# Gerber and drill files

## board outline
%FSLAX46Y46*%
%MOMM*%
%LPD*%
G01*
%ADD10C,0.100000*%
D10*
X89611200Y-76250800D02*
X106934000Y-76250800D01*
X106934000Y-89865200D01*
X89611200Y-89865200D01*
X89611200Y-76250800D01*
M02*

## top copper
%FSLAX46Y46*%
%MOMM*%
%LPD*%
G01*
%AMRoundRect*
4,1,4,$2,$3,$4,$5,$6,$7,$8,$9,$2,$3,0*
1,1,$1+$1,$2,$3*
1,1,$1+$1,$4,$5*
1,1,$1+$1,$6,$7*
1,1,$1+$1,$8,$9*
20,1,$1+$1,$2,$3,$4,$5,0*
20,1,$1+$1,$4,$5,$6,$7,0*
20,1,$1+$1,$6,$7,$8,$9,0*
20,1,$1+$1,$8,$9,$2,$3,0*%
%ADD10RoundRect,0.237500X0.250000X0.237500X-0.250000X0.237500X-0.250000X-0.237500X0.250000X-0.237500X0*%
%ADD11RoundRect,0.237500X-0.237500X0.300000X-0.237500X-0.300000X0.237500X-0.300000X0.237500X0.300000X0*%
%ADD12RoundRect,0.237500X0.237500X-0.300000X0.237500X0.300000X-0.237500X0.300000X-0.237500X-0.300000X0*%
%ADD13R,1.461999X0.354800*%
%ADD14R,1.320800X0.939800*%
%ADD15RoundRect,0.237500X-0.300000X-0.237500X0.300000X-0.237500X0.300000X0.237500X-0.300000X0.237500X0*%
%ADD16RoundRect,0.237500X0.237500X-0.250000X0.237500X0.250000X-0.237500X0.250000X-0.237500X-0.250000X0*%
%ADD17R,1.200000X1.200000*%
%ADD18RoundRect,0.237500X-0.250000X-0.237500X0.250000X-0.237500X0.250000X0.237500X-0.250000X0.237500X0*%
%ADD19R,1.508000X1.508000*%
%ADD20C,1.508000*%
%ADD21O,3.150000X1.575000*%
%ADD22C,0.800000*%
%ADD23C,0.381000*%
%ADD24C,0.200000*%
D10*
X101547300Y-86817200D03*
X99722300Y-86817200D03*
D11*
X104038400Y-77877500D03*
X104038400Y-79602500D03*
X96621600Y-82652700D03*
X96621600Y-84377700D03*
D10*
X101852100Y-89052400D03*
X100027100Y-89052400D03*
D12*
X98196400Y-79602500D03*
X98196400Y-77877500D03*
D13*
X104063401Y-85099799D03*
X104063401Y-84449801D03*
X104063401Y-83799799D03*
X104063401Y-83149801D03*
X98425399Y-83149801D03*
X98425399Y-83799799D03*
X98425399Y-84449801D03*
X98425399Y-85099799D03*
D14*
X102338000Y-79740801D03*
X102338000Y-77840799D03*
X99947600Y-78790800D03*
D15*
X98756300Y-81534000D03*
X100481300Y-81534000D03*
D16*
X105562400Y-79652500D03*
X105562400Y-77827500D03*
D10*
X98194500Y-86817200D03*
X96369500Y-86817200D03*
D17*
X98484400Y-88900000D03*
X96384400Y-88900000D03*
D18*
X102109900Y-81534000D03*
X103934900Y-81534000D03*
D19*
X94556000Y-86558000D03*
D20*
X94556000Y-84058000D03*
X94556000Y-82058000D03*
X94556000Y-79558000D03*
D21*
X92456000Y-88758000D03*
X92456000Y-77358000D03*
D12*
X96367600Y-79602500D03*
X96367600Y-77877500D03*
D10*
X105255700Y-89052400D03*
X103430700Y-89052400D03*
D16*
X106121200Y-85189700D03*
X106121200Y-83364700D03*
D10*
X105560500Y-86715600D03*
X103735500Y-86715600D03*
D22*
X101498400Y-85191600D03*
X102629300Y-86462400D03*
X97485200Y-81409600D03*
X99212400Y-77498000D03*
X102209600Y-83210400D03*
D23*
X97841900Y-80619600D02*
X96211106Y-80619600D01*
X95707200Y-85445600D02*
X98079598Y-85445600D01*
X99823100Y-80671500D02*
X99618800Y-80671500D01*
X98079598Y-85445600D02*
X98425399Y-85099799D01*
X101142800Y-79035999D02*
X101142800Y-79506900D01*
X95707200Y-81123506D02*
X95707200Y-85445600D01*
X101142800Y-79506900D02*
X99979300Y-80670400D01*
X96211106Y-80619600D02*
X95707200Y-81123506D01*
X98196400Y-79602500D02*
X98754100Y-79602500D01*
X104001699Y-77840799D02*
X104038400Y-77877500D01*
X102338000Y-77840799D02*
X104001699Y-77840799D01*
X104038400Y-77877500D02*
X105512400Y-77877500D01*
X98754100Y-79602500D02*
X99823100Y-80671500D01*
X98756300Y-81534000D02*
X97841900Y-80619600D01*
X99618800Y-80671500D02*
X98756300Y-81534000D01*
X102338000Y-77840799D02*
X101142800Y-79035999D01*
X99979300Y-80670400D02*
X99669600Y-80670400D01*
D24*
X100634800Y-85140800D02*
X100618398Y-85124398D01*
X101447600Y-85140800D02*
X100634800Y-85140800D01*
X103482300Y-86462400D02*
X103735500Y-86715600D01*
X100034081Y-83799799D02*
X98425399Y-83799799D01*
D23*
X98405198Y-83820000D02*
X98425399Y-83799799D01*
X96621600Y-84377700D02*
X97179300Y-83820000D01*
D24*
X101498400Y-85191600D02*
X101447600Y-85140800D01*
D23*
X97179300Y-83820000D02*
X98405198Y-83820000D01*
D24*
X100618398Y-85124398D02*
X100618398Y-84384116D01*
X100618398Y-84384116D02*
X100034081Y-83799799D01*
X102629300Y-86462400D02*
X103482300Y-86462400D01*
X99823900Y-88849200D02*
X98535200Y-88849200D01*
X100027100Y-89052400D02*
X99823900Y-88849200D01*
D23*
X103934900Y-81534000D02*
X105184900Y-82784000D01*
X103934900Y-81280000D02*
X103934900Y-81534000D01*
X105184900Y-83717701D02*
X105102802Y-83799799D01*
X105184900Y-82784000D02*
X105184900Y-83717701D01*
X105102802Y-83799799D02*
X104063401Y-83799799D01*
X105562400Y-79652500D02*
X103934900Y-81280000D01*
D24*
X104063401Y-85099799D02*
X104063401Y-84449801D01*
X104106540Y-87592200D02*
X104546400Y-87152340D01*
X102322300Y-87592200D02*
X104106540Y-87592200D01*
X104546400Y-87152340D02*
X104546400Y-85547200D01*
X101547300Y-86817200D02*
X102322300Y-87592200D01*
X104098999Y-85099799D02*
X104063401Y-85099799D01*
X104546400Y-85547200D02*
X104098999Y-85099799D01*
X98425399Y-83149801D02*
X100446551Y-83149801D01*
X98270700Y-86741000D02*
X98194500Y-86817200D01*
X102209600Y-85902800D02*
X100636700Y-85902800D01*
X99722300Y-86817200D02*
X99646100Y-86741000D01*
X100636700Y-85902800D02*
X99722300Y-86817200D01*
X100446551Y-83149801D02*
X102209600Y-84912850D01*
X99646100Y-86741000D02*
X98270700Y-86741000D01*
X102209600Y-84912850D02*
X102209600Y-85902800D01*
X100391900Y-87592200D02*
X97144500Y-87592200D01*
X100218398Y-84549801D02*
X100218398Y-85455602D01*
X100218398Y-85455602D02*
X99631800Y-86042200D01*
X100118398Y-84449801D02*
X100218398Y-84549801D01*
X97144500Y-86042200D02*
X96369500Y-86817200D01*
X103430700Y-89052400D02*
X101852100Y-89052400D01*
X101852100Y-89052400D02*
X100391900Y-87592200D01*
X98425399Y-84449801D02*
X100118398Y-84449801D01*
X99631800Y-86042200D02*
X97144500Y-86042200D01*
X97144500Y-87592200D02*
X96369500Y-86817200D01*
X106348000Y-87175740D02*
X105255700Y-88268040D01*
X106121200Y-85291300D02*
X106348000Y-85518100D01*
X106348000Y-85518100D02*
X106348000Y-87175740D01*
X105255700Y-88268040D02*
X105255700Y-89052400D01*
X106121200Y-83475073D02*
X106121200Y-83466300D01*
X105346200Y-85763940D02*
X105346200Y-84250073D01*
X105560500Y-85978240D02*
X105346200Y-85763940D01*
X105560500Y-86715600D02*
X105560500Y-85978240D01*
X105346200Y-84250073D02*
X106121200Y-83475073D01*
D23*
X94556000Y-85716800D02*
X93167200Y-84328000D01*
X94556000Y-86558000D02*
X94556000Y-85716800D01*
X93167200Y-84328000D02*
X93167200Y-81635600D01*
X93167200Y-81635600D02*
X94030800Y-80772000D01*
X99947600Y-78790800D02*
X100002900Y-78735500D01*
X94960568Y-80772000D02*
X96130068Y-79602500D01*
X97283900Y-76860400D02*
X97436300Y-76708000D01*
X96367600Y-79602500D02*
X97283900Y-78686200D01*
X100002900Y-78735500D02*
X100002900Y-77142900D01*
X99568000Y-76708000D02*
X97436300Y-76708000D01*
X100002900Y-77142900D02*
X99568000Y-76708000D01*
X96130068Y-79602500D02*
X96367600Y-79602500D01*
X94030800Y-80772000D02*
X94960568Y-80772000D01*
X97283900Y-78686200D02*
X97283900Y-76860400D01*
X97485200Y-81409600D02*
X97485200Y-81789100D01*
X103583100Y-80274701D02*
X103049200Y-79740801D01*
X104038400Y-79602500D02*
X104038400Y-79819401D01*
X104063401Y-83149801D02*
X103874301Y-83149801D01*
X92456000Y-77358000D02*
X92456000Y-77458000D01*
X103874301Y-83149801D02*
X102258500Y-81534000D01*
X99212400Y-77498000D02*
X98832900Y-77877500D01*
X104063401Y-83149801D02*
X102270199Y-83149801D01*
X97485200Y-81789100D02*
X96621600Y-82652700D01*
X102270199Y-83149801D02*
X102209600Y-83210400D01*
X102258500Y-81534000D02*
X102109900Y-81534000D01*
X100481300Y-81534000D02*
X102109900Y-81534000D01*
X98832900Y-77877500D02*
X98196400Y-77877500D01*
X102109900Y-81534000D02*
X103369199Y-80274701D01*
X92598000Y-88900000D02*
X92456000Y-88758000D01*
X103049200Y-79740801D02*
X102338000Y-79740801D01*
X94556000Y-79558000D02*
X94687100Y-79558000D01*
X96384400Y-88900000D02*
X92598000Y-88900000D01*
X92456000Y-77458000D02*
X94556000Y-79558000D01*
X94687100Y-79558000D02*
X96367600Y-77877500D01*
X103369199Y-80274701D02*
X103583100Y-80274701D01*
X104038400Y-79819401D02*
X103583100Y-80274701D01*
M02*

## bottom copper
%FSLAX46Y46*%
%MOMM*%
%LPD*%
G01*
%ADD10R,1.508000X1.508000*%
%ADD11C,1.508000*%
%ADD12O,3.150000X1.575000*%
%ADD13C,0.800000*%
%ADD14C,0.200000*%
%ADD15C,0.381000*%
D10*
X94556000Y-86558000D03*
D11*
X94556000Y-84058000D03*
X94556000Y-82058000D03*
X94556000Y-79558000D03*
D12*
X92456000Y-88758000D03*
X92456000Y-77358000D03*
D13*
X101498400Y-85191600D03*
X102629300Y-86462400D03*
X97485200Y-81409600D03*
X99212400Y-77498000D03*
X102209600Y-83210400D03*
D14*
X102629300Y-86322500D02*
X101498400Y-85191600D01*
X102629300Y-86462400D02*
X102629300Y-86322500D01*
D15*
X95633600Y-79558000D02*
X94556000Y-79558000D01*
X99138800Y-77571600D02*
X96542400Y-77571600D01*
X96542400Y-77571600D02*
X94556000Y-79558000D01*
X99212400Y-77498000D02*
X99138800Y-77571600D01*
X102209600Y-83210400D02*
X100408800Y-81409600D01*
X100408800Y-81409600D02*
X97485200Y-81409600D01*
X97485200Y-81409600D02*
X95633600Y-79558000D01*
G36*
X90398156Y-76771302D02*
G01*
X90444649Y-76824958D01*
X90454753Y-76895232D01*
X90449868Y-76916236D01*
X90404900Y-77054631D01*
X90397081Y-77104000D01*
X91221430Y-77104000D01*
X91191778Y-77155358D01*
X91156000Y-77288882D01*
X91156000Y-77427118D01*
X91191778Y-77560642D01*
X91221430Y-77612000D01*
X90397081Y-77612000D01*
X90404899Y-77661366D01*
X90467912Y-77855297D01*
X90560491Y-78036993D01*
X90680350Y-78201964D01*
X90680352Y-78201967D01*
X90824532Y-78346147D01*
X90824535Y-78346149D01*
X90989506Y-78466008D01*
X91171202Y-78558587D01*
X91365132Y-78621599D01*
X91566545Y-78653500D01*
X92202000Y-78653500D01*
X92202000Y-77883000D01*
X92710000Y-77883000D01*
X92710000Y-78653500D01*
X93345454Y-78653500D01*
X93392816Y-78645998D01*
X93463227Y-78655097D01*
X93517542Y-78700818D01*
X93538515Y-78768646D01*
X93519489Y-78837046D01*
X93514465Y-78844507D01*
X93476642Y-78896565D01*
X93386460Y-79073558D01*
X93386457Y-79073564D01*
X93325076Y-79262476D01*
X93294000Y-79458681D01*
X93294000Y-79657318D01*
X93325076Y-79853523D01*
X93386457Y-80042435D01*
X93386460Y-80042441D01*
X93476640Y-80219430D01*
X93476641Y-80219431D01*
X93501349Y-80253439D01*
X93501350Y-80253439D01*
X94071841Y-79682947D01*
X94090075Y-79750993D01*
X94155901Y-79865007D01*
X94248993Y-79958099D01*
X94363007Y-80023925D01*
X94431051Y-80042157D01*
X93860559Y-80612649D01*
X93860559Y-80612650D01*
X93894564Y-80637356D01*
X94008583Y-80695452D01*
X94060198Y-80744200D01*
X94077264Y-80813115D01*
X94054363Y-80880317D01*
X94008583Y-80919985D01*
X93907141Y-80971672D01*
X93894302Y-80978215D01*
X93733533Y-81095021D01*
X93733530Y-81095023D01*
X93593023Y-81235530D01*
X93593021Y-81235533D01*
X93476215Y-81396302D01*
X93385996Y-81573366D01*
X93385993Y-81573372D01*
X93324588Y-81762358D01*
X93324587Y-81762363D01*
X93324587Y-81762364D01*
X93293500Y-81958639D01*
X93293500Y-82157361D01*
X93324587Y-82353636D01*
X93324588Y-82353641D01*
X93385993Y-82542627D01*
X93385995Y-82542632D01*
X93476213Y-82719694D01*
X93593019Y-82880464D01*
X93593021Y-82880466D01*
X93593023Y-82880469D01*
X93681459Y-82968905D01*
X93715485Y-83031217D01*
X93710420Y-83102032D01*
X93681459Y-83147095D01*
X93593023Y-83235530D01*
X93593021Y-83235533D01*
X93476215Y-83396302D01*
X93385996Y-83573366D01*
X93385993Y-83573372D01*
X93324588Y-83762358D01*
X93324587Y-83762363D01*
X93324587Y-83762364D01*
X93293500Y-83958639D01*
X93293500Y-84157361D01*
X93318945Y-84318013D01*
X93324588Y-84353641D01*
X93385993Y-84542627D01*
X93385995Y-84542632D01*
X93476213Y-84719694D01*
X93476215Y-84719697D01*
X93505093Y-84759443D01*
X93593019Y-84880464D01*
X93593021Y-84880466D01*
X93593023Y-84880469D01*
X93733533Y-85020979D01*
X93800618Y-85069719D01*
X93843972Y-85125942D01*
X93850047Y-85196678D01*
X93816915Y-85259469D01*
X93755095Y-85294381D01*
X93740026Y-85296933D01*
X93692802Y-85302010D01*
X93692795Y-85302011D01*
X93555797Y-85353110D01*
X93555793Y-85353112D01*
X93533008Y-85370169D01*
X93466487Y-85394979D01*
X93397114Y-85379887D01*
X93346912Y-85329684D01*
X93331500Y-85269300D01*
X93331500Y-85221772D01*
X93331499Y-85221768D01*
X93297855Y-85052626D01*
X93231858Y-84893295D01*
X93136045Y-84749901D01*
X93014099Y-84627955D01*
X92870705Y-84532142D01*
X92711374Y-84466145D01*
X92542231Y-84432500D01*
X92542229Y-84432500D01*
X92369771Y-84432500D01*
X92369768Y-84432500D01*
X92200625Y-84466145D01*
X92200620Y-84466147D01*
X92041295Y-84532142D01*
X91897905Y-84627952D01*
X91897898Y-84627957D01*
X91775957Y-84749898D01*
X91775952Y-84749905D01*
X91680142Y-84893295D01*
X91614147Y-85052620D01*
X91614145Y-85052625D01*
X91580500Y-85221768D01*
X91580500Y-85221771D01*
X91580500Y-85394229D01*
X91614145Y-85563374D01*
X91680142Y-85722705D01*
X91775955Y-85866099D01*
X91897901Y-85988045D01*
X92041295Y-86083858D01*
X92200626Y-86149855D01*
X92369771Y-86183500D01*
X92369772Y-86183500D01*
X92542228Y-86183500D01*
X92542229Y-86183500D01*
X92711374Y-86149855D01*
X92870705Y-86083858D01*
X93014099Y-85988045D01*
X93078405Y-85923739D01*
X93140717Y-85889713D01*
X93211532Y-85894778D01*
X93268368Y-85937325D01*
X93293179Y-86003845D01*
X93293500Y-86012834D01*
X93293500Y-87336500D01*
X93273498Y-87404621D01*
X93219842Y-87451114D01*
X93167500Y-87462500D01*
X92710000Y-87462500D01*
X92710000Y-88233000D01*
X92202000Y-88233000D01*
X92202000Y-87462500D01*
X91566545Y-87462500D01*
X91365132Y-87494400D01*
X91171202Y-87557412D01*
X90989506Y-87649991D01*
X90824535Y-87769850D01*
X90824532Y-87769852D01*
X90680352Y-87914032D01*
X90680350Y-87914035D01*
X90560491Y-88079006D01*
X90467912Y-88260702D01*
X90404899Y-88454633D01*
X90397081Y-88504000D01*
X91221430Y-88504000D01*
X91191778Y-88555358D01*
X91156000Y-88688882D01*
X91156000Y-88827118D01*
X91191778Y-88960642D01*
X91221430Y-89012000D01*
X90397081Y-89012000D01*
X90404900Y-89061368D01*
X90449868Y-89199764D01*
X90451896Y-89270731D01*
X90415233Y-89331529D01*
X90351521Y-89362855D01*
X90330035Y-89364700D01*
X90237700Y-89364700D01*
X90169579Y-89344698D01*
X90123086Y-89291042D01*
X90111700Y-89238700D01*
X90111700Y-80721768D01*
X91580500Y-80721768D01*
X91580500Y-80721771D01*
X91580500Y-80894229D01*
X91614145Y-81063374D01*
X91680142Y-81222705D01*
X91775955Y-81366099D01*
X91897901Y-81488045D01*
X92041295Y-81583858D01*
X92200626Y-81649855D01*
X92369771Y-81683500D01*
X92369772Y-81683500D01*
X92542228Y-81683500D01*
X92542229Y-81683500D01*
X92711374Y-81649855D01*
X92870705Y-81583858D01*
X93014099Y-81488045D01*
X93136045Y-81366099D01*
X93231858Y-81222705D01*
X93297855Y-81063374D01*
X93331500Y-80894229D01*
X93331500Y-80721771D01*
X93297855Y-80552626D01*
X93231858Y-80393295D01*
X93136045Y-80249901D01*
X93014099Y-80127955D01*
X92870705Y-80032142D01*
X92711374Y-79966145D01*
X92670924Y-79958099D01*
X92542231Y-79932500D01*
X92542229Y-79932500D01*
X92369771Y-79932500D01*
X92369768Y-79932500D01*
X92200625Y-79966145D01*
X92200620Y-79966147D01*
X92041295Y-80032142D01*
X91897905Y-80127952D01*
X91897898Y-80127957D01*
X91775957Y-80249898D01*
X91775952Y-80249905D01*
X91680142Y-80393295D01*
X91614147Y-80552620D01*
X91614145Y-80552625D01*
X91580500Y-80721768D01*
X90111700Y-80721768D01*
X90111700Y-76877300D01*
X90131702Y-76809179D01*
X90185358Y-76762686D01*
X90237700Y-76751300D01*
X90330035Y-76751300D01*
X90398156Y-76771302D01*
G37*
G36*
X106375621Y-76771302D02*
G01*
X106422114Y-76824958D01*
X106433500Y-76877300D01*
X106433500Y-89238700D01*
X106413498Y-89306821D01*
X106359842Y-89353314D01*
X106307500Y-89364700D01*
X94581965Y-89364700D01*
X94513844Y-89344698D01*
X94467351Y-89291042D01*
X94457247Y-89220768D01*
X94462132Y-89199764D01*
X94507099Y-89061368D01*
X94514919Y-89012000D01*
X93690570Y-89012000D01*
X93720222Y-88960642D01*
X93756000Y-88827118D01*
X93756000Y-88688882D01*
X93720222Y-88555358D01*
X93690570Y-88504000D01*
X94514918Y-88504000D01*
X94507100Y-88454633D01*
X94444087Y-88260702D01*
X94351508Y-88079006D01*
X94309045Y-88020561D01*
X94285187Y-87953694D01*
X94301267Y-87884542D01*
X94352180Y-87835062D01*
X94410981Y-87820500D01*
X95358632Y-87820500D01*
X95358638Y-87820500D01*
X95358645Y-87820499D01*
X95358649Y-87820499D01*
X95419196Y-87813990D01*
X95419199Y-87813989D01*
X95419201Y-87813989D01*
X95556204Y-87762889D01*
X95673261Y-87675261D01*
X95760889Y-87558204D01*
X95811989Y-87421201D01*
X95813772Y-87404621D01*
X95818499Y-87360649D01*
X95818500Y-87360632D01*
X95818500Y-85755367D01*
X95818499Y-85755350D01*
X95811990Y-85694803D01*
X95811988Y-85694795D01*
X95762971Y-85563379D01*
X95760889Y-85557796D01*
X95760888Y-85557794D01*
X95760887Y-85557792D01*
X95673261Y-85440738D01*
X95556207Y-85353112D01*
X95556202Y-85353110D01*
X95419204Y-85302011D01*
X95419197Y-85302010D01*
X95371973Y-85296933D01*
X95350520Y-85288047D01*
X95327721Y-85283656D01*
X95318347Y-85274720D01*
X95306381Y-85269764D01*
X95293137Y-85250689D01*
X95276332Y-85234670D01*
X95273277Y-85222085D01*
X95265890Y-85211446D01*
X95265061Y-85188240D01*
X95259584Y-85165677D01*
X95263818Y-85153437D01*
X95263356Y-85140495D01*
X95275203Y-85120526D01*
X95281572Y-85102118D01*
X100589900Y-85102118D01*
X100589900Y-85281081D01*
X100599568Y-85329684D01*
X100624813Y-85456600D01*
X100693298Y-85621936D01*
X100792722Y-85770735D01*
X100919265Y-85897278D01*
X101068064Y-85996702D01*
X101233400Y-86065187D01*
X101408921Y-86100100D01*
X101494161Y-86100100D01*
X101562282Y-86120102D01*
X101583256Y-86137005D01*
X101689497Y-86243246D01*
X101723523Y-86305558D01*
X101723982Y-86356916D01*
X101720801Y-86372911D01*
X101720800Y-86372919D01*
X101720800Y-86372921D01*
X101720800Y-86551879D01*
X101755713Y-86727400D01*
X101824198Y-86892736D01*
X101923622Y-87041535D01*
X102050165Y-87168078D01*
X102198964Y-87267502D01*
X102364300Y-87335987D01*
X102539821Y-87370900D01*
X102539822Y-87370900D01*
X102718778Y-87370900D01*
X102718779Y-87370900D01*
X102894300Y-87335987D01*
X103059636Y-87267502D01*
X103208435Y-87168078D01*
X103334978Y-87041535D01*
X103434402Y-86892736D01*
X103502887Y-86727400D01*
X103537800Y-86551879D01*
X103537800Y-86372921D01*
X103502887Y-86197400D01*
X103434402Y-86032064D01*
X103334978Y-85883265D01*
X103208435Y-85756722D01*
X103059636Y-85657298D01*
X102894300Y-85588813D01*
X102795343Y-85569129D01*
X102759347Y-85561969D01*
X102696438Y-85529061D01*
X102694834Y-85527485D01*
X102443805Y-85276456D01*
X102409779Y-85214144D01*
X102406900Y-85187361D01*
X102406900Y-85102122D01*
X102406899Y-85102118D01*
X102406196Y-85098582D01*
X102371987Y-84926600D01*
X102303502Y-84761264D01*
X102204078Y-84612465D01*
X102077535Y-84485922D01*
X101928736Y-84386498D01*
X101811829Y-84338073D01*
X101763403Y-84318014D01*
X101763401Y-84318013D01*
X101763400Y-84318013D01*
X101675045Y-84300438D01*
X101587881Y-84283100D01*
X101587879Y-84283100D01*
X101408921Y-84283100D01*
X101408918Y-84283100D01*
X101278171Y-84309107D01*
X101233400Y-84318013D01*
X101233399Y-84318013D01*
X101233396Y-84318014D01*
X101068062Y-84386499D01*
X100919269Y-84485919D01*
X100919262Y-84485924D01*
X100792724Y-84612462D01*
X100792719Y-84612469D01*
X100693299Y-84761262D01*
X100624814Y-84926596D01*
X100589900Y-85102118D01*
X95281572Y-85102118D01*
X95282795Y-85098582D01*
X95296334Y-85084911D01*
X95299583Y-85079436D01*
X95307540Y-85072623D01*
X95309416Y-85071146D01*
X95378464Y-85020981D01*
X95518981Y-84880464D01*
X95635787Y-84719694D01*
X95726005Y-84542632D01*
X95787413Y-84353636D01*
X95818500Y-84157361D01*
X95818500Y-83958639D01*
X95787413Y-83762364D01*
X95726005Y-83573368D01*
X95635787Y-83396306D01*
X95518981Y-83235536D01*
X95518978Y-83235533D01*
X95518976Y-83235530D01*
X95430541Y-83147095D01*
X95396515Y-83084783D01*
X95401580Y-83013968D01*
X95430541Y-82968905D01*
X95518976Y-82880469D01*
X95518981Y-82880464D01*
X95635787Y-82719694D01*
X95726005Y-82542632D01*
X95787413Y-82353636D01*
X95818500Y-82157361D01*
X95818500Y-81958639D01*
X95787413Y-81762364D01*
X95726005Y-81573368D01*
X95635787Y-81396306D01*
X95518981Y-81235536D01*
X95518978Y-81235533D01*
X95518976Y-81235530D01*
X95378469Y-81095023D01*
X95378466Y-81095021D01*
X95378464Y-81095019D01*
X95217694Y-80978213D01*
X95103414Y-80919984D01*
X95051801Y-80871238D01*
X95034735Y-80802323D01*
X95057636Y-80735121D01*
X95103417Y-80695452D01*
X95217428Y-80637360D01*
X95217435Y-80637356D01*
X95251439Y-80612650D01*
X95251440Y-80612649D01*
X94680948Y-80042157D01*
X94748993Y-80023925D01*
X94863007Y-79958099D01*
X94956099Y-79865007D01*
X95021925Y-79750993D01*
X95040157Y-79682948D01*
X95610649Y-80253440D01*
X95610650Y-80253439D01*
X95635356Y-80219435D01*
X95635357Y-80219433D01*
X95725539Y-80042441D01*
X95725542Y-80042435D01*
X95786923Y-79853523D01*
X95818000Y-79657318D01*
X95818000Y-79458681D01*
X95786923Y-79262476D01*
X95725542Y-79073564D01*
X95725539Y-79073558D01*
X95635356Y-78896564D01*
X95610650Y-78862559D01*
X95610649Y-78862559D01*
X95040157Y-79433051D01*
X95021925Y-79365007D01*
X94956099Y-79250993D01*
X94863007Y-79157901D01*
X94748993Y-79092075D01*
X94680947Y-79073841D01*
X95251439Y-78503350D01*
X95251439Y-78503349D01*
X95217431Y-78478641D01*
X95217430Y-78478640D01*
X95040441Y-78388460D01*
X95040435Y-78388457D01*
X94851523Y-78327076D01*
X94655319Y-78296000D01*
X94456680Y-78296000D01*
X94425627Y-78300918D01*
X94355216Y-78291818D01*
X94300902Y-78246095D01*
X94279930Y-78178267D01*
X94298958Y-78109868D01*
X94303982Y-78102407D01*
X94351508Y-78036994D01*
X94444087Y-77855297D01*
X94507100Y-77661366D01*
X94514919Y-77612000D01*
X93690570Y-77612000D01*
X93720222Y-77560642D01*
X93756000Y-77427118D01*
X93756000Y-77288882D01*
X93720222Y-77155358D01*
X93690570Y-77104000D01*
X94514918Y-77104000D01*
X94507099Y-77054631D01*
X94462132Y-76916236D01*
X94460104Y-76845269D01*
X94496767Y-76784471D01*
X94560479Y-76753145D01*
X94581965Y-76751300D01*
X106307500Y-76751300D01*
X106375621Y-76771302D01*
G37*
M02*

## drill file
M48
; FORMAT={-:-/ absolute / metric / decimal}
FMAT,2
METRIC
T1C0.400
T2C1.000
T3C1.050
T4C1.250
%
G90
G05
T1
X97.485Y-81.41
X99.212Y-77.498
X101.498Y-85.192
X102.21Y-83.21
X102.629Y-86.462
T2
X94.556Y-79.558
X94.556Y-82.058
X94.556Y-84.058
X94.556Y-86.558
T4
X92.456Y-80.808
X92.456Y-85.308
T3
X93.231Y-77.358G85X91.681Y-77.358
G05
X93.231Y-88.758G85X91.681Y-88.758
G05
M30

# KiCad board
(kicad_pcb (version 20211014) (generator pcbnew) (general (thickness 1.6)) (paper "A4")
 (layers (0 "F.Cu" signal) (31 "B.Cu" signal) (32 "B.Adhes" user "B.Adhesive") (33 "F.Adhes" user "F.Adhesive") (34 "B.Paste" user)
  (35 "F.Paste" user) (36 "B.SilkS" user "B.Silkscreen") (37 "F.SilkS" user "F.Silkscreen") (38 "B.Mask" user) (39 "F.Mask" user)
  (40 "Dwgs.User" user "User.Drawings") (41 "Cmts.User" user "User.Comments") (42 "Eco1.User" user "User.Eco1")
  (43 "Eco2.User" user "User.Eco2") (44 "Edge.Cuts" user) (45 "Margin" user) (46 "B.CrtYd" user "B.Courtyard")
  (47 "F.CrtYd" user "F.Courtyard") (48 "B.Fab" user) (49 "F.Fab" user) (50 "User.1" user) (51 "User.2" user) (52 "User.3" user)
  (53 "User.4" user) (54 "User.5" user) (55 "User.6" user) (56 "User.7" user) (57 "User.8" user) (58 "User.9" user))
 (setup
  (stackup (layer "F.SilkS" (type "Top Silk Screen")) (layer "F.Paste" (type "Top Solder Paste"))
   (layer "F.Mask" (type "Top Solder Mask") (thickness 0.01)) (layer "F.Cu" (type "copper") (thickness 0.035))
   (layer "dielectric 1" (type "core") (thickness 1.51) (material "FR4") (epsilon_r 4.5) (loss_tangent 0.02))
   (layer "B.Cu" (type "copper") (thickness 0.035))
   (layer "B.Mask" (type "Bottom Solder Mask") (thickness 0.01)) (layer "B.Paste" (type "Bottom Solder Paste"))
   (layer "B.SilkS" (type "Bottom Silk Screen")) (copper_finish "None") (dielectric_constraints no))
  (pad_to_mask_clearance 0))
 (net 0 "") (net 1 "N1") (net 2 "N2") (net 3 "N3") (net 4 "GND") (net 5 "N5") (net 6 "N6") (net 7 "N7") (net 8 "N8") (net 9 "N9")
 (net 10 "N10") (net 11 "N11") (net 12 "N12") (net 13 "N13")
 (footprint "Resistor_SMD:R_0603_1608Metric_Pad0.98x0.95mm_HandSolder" (layer "F.Cu") (at 100.6348 86.8172 180)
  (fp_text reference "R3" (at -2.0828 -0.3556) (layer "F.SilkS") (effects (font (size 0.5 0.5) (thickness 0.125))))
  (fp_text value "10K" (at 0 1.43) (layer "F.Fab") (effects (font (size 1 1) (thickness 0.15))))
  (pad "1" smd roundrect (at -0.9125 0 180) (size 0.975 0.95) (layers "F.Cu" "F.Paste" "F.Mask") (roundrect_rratio 0.25) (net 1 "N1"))
  (pad "2" smd roundrect (at 0.9125 0 180) (size 0.975 0.95) (layers "F.Cu" "F.Paste" "F.Mask") (roundrect_rratio 0.25) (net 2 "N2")))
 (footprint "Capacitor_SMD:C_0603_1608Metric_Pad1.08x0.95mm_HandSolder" (layer "F.Cu") (at 104.0384 78.74 -90)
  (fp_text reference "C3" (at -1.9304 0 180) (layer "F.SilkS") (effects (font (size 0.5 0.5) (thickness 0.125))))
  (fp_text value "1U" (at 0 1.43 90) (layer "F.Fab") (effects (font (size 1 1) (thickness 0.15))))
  (pad "1" smd roundrect (at -0.8625 0 270) (size 1.075 0.95) (layers "F.Cu" "F.Paste" "F.Mask") (roundrect_rratio 0.25) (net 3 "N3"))
  (pad "2" smd roundrect (at 0.8625 0 270) (size 1.075 0.95) (layers "F.Cu" "F.Paste" "F.Mask") (roundrect_rratio 0.25) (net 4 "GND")))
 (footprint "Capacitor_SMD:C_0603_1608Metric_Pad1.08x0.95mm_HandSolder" (layer "F.Cu") (at 96.6216 83.5152 -90)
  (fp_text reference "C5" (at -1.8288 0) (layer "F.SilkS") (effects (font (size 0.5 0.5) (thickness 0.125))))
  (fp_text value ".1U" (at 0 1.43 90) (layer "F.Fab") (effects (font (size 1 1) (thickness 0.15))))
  (pad "1" smd roundrect (at -0.8625 0 270) (size 1.075 0.95) (layers "F.Cu" "F.Paste" "F.Mask") (roundrect_rratio 0.25) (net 4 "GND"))
  (pad "2" smd roundrect (at 0.8625 0 270) (size 1.075 0.95) (layers "F.Cu" "F.Paste" "F.Mask") (roundrect_rratio 0.25) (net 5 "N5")))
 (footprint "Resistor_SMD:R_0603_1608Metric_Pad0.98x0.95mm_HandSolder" (layer "F.Cu") (at 100.9396 89.0524 180)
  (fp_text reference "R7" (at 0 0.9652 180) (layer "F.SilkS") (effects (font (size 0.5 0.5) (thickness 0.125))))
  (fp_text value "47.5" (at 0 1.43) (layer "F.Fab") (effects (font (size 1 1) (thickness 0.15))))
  (pad "1" smd roundrect (at -0.9125 0 180) (size 0.975 0.95) (layers "F.Cu" "F.Paste" "F.Mask") (roundrect_rratio 0.25) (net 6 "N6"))
  (pad "2" smd roundrect (at 0.9125 0 180) (size 0.975 0.95) (layers "F.Cu" "F.Paste" "F.Mask") (roundrect_rratio 0.25) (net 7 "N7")))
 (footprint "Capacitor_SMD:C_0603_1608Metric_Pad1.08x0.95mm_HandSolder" (layer "F.Cu") (at 98.1964 78.74 90)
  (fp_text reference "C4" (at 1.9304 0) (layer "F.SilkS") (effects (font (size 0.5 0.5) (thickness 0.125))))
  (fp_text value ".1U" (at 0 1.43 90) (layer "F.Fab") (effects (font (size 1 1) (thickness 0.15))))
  (pad "1" smd roundrect (at -0.8625 0 90) (size 1.075 0.95) (layers "F.Cu" "F.Paste" "F.Mask") (roundrect_rratio 0.25) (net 3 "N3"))
  (pad "2" smd roundrect (at 0.8625 0 90) (size 1.075 0.95) (layers "F.Cu" "F.Paste" "F.Mask") (roundrect_rratio 0.25) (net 4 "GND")))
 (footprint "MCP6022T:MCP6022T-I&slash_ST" (layer "F.Cu") (at 101.2444 84.1248 180)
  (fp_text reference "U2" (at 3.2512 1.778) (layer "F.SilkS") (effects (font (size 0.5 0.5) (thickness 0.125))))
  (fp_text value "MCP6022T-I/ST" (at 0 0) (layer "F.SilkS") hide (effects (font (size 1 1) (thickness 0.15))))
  (pad "1" smd rect (at -2.819001 -0.974999 180) (size 1.461999 0.3548) (layers "F.Cu" "F.Paste" "F.Mask") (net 1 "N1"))
  (pad "2" smd rect (at -2.819001 -0.325001 180) (size 1.461999 0.3548) (layers "F.Cu" "F.Paste" "F.Mask") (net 1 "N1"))
  (pad "3" smd rect (at -2.819001 0.325001 180) (size 1.461999 0.3548) (layers "F.Cu" "F.Paste" "F.Mask") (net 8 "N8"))
  (pad "4" smd rect (at -2.819001 0.974999 180) (size 1.461999 0.3548) (layers "F.Cu" "F.Paste" "F.Mask") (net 4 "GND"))
  (pad "5" smd rect (at 2.819001 0.974999 180) (size 1.461999 0.3548) (layers "F.Cu" "F.Paste" "F.Mask") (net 2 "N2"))
  (pad "6" smd rect (at 2.819001 0.325001 180) (size 1.461999 0.3548) (layers "F.Cu" "F.Paste" "F.Mask") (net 5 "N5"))
  (pad "7" smd rect (at 2.819001 -0.325001 180) (size 1.461999 0.3548) (layers "F.Cu" "F.Paste" "F.Mask") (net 6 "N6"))
  (pad "8" smd rect (at 2.819001 -0.974999 180) (size 1.461999 0.3548) (layers "F.Cu" "F.Paste" "F.Mask") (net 3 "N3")))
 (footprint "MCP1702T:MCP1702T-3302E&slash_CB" (layer "F.Cu") (at 101.1428 78.7908 90)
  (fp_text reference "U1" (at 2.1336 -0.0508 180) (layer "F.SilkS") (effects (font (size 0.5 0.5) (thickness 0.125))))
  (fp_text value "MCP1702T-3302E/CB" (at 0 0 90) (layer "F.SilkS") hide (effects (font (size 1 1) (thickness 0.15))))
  (pad "1" smd rect (at -0.950001 1.1952 90) (size 0.9398 1.3208) (layers "F.Cu" "F.Paste" "F.Mask") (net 4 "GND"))
  (pad "2" smd rect (at 0.950001 1.1952 90) (size 0.9398 1.3208) (layers "F.Cu" "F.Paste" "F.Mask") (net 3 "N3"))
  (pad "3" smd rect (at 0 -1.1952 90) (size 0.9398 1.3208) (layers "F.Cu" "F.Paste" "F.Mask") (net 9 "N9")))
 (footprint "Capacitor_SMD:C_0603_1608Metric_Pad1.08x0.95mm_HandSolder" (layer "F.Cu") (at 99.6188 81.534)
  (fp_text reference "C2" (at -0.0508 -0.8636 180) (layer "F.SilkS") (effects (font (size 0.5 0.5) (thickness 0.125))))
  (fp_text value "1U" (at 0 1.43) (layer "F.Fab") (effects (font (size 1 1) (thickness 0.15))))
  (pad "1" smd roundrect (at -0.8625 0) (size 1.075 0.95) (layers "F.Cu" "F.Paste" "F.Mask") (roundrect_rratio 0.25) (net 3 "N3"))
  (pad "2" smd roundrect (at 0.8625 0) (size 1.075 0.95) (layers "F.Cu" "F.Paste" "F.Mask") (roundrect_rratio 0.25) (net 4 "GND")))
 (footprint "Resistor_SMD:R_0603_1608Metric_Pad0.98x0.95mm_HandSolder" (layer "F.Cu") (at 105.5624 78.74 90)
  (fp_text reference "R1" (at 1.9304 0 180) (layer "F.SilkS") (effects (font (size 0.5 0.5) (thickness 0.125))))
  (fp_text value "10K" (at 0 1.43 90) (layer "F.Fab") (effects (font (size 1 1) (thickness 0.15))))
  (pad "1" smd roundrect (at -0.9125 0 90) (size 0.975 0.95) (layers "F.Cu" "F.Paste" "F.Mask") (roundrect_rratio 0.25) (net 8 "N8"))
  (pad "2" smd roundrect (at 0.9125 0 90) (size 0.975 0.95) (layers "F.Cu" "F.Paste" "F.Mask") (roundrect_rratio 0.25) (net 3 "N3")))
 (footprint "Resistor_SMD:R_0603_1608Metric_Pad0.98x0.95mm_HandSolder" (layer "F.Cu") (at 97.282 86.8172 180)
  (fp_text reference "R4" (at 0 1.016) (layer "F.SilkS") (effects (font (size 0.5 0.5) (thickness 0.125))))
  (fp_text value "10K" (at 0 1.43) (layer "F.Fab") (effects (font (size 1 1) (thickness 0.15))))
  (pad "1" smd roundrect (at -0.9125 0 180) (size 0.975 0.95) (layers "F.Cu" "F.Paste" "F.Mask") (roundrect_rratio 0.25) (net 2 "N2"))
  (pad "2" smd roundrect (at 0.9125 0 180) (size 0.975 0.95) (layers "F.Cu" "F.Paste" "F.Mask") (roundrect_rratio 0.25) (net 6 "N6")))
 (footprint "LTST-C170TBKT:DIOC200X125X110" (layer "F.Cu") (at 97.4344 88.9)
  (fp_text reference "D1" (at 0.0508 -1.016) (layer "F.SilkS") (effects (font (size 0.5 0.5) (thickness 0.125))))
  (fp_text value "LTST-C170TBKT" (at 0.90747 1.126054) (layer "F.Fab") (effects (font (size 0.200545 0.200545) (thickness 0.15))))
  (pad "+" smd rect locked (at 1.05 0) (size 1.2 1.2) (layers "F.Cu" "F.Paste" "F.Mask") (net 7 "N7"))
  (pad "-" smd rect locked (at -1.05 0) (size 1.2 1.2) (layers "F.Cu" "F.Paste" "F.Mask") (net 4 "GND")))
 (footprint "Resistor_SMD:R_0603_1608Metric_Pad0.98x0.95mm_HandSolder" (layer "F.Cu") (at 103.0224 81.534)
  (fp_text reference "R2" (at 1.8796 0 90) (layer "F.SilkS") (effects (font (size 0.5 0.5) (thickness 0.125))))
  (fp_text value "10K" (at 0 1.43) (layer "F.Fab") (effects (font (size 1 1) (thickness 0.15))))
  (pad "1" smd roundrect (at -0.9125 0) (size 0.975 0.95) (layers "F.Cu" "F.Paste" "F.Mask") (roundrect_rratio 0.25) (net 4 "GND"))
  (pad "2" smd roundrect (at 0.9125 0) (size 0.975 0.95) (layers "F.Cu" "F.Paste" "F.Mask") (roundrect_rratio 0.25) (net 8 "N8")))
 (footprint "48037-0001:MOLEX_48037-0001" (layer "F.Cu") (at 92.456 83.058 -90)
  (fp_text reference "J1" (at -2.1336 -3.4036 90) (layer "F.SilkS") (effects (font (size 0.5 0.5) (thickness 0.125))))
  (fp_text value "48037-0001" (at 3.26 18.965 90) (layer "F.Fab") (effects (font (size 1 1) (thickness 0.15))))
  (pad "" np_thru_hole circle (at -2.25 0 270) (size 1.25 1.25) (drill 1.25) (layers *.Cu *.Mask))
  (pad "" np_thru_hole circle (at 2.25 0 270) (size 1.25 1.25) (drill 1.25) (layers *.Cu *.Mask))
  (pad "1" thru_hole rect (at 3.5 -2.1 270) (size 1.508 1.508) (drill 1) (layers *.Cu *.Mask) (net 9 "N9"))
  (pad "2" thru_hole circle (at 1 -2.1 270) (size 1.508 1.508) (drill 1) (layers *.Cu *.Mask) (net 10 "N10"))
  (pad "3" thru_hole circle (at -1 -2.1 270) (size 1.508 1.508) (drill 1) (layers *.Cu *.Mask) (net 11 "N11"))
  (pad "4" thru_hole circle (at -3.5 -2.1 270) (size 1.508 1.508) (drill 1) (layers *.Cu *.Mask) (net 4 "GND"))
  (pad "S1" thru_hole oval (at 5.7 0 270) (size 1.575 3.15) (drill oval 1.05 2.6) (layers *.Cu *.Mask) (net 4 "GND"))
  (pad "S2" thru_hole oval (at -5.7 0 270) (size 1.575 3.15) (drill oval 1.05 2.6) (layers *.Cu *.Mask) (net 4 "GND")))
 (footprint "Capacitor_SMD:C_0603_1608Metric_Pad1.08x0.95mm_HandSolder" (layer "F.Cu") (at 96.3676 78.74 90)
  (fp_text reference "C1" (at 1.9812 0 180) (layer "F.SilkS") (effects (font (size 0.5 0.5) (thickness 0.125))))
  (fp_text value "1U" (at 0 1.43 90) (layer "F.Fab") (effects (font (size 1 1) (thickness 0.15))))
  (pad "1" smd roundrect (at -0.8625 0 90) (size 1.075 0.95) (layers "F.Cu" "F.Paste" "F.Mask") (roundrect_rratio 0.25) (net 9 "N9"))
  (pad "2" smd roundrect (at 0.8625 0 90) (size 1.075 0.95) (layers "F.Cu" "F.Paste" "F.Mask") (roundrect_rratio 0.25) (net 4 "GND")))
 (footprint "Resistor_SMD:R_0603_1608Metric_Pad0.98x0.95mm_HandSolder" (layer "F.Cu") (at 104.3432 89.0524 180)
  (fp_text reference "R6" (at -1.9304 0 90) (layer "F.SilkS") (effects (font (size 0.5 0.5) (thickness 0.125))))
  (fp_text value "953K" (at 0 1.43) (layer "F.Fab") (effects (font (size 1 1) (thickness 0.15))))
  (pad "1" smd roundrect (at -0.9125 0 180) (size 0.975 0.95) (layers "F.Cu" "F.Paste" "F.Mask") (roundrect_rratio 0.25) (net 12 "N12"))
  (pad "2" smd roundrect (at 0.9125 0 180) (size 0.975 0.95) (layers "F.Cu" "F.Paste" "F.Mask") (roundrect_rratio 0.25) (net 6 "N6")))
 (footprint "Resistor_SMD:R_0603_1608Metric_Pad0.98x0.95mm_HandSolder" (layer "F.Cu") (at 106.1212 84.2772 90)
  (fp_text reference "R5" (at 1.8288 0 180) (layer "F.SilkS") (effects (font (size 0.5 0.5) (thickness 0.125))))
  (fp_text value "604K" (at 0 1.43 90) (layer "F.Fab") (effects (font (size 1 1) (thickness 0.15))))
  (pad "1" smd roundrect (at -0.9125 0 90) (size 0.975 0.95) (layers "F.Cu" "F.Paste" "F.Mask") (roundrect_rratio 0.25) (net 12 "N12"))
  (pad "2" smd roundrect (at 0.9125 0 90) (size 0.975 0.95) (layers "F.Cu" "F.Paste" "F.Mask") (roundrect_rratio 0.25) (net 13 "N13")))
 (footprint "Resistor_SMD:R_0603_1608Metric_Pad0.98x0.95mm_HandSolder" (layer "F.Cu") (at 104.648 86.7156 180)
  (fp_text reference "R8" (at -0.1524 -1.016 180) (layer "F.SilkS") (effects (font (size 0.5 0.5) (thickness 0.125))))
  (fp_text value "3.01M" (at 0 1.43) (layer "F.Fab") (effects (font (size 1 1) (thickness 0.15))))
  (pad "1" smd roundrect (at -0.9125 0 180) (size 0.975 0.95) (layers "F.Cu" "F.Paste" "F.Mask") (roundrect_rratio 0.25) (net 13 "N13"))
  (pad "2" smd roundrect (at 0.9125 0 180) (size 0.975 0.95) (layers "F.Cu" "F.Paste" "F.Mask") (roundrect_rratio 0.25) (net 5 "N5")))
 (gr_rect (start 89.6112 76.2508) (end 106.934 89.8652) (layer "Edge.Cuts") (width 0.1) (fill none))
 (segment (start 97.8419 80.6196) (end 96.211106 80.6196) (width 0.381) (layer "F.Cu") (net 3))
 (segment (start 95.7072 85.4456) (end 98.079598 85.4456) (width 0.381) (layer "F.Cu") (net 3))
 (segment (start 99.8231 80.6715) (end 99.6188 80.6715) (width 0.381) (layer "F.Cu") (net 3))
 (segment (start 98.079598 85.4456) (end 98.425399 85.099799) (width 0.381) (layer "F.Cu") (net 3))
 (segment (start 101.1428 79.035999) (end 101.1428 79.5069) (width 0.381) (layer "F.Cu") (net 3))
 (segment (start 95.7072 81.123506) (end 95.7072 85.4456) (width 0.381) (layer "F.Cu") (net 3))
 (segment (start 101.1428 79.5069) (end 99.9793 80.6704) (width 0.381) (layer "F.Cu") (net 3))
 (segment (start 96.211106 80.6196) (end 95.7072 81.123506) (width 0.381) (layer "F.Cu") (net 3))
 (segment (start 98.1964 79.6025) (end 98.7541 79.6025) (width 0.381) (layer "F.Cu") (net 3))
 (segment (start 104.001699 77.840799) (end 104.0384 77.8775) (width 0.381) (layer "F.Cu") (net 3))
 (segment (start 102.338 77.840799) (end 104.001699 77.840799) (width 0.381) (layer "F.Cu") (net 3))
 (segment (start 104.0384 77.8775) (end 105.5124 77.8775) (width 0.381) (layer "F.Cu") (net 3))
 (segment (start 98.7541 79.6025) (end 99.8231 80.6715) (width 0.381) (layer "F.Cu") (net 3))
 (segment (start 98.7563 81.534) (end 97.8419 80.6196) (width 0.381) (layer "F.Cu") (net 3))
 (segment (start 99.6188 80.6715) (end 98.7563 81.534) (width 0.381) (layer "F.Cu") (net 3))
 (segment (start 102.338 77.840799) (end 101.1428 79.035999) (width 0.381) (layer "F.Cu") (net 3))
 (segment (start 99.9793 80.6704) (end 99.6696 80.6704) (width 0.381) (layer "F.Cu") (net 3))
 (segment (start 100.6348 85.1408) (end 100.618398 85.124398) (width 0.2) (layer "F.Cu") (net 5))
 (segment (start 101.4476 85.1408) (end 100.6348 85.1408) (width 0.2) (layer "F.Cu") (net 5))
 (segment (start 103.4823 86.4624) (end 103.7355 86.7156) (width 0.2) (layer "F.Cu") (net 5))
 (segment (start 100.034081 83.799799) (end 98.425399 83.799799) (width 0.2) (layer "F.Cu") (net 5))
 (segment (start 98.405198 83.82) (end 98.425399 83.799799) (width 0.381) (layer "F.Cu") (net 5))
 (segment (start 96.6216 84.3777) (end 97.1793 83.82) (width 0.381) (layer "F.Cu") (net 5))
 (segment (start 101.4984 85.1916) (end 101.4476 85.1408) (width 0.2) (layer "F.Cu") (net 5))
 (segment (start 97.1793 83.82) (end 98.405198 83.82) (width 0.381) (layer "F.Cu") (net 5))
 (segment (start 100.618398 85.124398) (end 100.618398 84.384116) (width 0.2) (layer "F.Cu") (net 5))
 (segment (start 100.618398 84.384116) (end 100.034081 83.799799) (width 0.2) (layer "F.Cu") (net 5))
 (segment (start 102.6293 86.4624) (end 103.4823 86.4624) (width 0.2) (layer "F.Cu") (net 5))
 (via (at 101.4984 85.1916) (size 0.8) (drill 0.4) (layers "F.Cu" "B.Cu") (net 5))
 (via (at 102.6293 86.4624) (size 0.8) (drill 0.4) (layers "F.Cu" "B.Cu") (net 5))
 (segment (start 102.6293 86.3225) (end 101.4984 85.1916) (width 0.2) (layer "B.Cu") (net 5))
 (segment (start 102.6293 86.4624) (end 102.6293 86.3225) (width 0.2) (layer "B.Cu") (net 5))
 (segment (start 99.8239 88.8492) (end 98.5352 88.8492) (width 0.2) (layer "F.Cu") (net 7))
 (segment (start 100.0271 89.0524) (end 99.8239 88.8492) (width 0.2) (layer "F.Cu") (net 7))
 (segment (start 103.9349 81.534) (end 105.1849 82.784) (width 0.381) (layer "F.Cu") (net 8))
 (segment (start 103.9349 81.28) (end 103.9349 81.534) (width 0.381) (layer "F.Cu") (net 8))
 (segment (start 105.1849 83.717701) (end 105.102802 83.799799) (width 0.381) (layer "F.Cu") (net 8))
 (segment (start 105.1849 82.784) (end 105.1849 83.717701) (width 0.381) (layer "F.Cu") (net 8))
 (segment (start 105.102802 83.799799) (end 104.063401 83.799799) (width 0.381) (layer "F.Cu") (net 8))
 (segment (start 105.5624 79.6525) (end 103.9349 81.28) (width 0.381) (layer "F.Cu") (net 8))
 (segment (start 104.063401 85.099799) (end 104.063401 84.449801) (width 0.2) (layer "F.Cu") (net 1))
 (segment (start 104.10654 87.5922) (end 104.5464 87.15234) (width 0.2) (layer "F.Cu") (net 1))
 (segment (start 102.3223 87.5922) (end 104.10654 87.5922) (width 0.2) (layer "F.Cu") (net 1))
 (segment (start 104.5464 87.15234) (end 104.5464 85.5472) (width 0.2) (layer "F.Cu") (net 1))
 (segment (start 101.5473 86.8172) (end 102.3223 87.5922) (width 0.2) (layer "F.Cu") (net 1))
 (segment (start 104.098999 85.099799) (end 104.063401 85.099799) (width 0.2) (layer "F.Cu") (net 1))
 (segment (start 104.5464 85.5472) (end 104.098999 85.099799) (width 0.2) (layer "F.Cu") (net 1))
 (segment (start 98.425399 83.149801) (end 100.446551 83.149801) (width 0.2) (layer "F.Cu") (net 2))
 (segment (start 98.2707 86.741) (end 98.1945 86.8172) (width 0.2) (layer "F.Cu") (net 2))
 (segment (start 102.2096 85.9028) (end 100.6367 85.9028) (width 0.2) (layer "F.Cu") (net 2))
 (segment (start 99.7223 86.8172) (end 99.6461 86.741) (width 0.2) (layer "F.Cu") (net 2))
 (segment (start 100.6367 85.9028) (end 99.7223 86.8172) (width 0.2) (layer "F.Cu") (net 2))
 (segment (start 100.446551 83.149801) (end 102.2096 84.91285) (width 0.2) (layer "F.Cu") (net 2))
 (segment (start 99.6461 86.741) (end 98.2707 86.741) (width 0.2) (layer "F.Cu") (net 2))
 (segment (start 102.2096 84.91285) (end 102.2096 85.9028) (width 0.2) (layer "F.Cu") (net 2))
 (segment (start 100.3919 87.5922) (end 97.1445 87.5922) (width 0.2) (layer "F.Cu") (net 6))
 (segment (start 100.218398 84.549801) (end 100.218398 85.455602) (width 0.2) (layer "F.Cu") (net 6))
 (segment (start 100.218398 85.455602) (end 99.6318 86.0422) (width 0.2) (layer "F.Cu") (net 6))
 (segment (start 100.118398 84.449801) (end 100.218398 84.549801) (width 0.2) (layer "F.Cu") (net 6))
 (segment (start 97.1445 86.0422) (end 96.3695 86.8172) (width 0.2) (layer "F.Cu") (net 6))
 (segment (start 103.4307 89.0524) (end 101.8521 89.0524) (width 0.2) (layer "F.Cu") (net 6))
 (segment (start 101.8521 89.0524) (end 100.3919 87.5922) (width 0.2) (layer "F.Cu") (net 6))
 (segment (start 98.425399 84.449801) (end 100.118398 84.449801) (width 0.2) (layer "F.Cu") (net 6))
 (segment (start 99.6318 86.0422) (end 97.1445 86.0422) (width 0.2) (layer "F.Cu") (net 6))
 (segment (start 97.1445 87.5922) (end 96.3695 86.8172) (width 0.2) (layer "F.Cu") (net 6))
 (segment (start 106.348 87.17574) (end 105.2557 88.26804) (width 0.2) (layer "F.Cu") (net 12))
 (segment (start 106.1212 85.2913) (end 106.348 85.5181) (width 0.2) (layer "F.Cu") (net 12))
 (segment (start 106.348 85.5181) (end 106.348 87.17574) (width 0.2) (layer "F.Cu") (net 12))
 (segment (start 105.2557 88.26804) (end 105.2557 89.0524) (width 0.2) (layer "F.Cu") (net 12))
 (segment (start 106.1212 83.475073) (end 106.1212 83.4663) (width 0.2) (layer "F.Cu") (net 13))
 (segment (start 105.3462 85.76394) (end 105.3462 84.250073) (width 0.2) (layer "F.Cu") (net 13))
 (segment (start 105.5605 85.97824) (end 105.3462 85.76394) (width 0.2) (layer "F.Cu") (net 13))
 (segment (start 105.5605 86.7156) (end 105.5605 85.97824) (width 0.2) (layer "F.Cu") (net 13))
 (segment (start 105.3462 84.250073) (end 106.1212 83.475073) (width 0.2) (layer "F.Cu") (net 13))
 (segment (start 94.556 85.7168) (end 93.1672 84.328) (width 0.381) (layer "F.Cu") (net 9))
 (segment (start 94.556 86.558) (end 94.556 85.7168) (width 0.381) (layer "F.Cu") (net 9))
 (segment (start 93.1672 84.328) (end 93.1672 81.6356) (width 0.381) (layer "F.Cu") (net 9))
 (segment (start 93.1672 81.6356) (end 94.0308 80.772) (width 0.381) (layer "F.Cu") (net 9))
 (segment (start 99.9476 78.7908) (end 100.0029 78.7355) (width 0.381) (layer "F.Cu") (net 9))
 (segment (start 94.960568 80.772) (end 96.130068 79.6025) (width 0.381) (layer "F.Cu") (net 9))
 (segment (start 97.2839 76.8604) (end 97.4363 76.708) (width 0.381) (layer "F.Cu") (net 9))
 (segment (start 96.3676 79.6025) (end 97.2839 78.6862) (width 0.381) (layer "F.Cu") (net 9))
 (segment (start 100.0029 78.7355) (end 100.0029 77.1429) (width 0.381) (layer "F.Cu") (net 9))
 (segment (start 99.568 76.708) (end 97.4363 76.708) (width 0.381) (layer "F.Cu") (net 9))
 (segment (start 100.0029 77.1429) (end 99.568 76.708) (width 0.381) (layer "F.Cu") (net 9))
 (segment (start 96.130068 79.6025) (end 96.3676 79.6025) (width 0.381) (layer "F.Cu") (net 9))
 (segment (start 94.0308 80.772) (end 94.960568 80.772) (width 0.381) (layer "F.Cu") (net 9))
 (segment (start 97.2839 78.6862) (end 97.2839 76.8604) (width 0.381) (layer "F.Cu") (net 9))
 (segment (start 97.4852 81.4096) (end 97.4852 81.7891) (width 0.381) (layer "F.Cu") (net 4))
 (segment (start 103.5831 80.274701) (end 103.0492 79.740801) (width 0.381) (layer "F.Cu") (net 4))
 (segment (start 104.0384 79.6025) (end 104.0384 79.819401) (width 0.381) (layer "F.Cu") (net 4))
 (segment (start 104.063401 83.149801) (end 103.874301 83.149801) (width 0.381) (layer "F.Cu") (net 4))
 (segment (start 92.456 77.358) (end 92.456 77.458) (width 0.381) (layer "F.Cu") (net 4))
 (segment (start 103.874301 83.149801) (end 102.2585 81.534) (width 0.381) (layer "F.Cu") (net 4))
 (segment (start 99.2124 77.498) (end 98.8329 77.8775) (width 0.381) (layer "F.Cu") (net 4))
 (segment (start 104.063401 83.149801) (end 102.270199 83.149801) (width 0.381) (layer "F.Cu") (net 4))
 (segment (start 97.4852 81.7891) (end 96.6216 82.6527) (width 0.381) (layer "F.Cu") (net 4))
 (segment (start 102.270199 83.149801) (end 102.2096 83.2104) (width 0.381) (layer "F.Cu") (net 4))
 (segment (start 102.2585 81.534) (end 102.1099 81.534) (width 0.381) (layer "F.Cu") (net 4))
 (segment (start 100.4813 81.534) (end 102.1099 81.534) (width 0.381) (layer "F.Cu") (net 4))
 (segment (start 98.8329 77.8775) (end 98.1964 77.8775) (width 0.381) (layer "F.Cu") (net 4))
 (segment (start 102.1099 81.534) (end 103.369199 80.274701) (width 0.381) (layer "F.Cu") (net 4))
 (segment (start 92.598 88.9) (end 92.456 88.758) (width 0.381) (layer "F.Cu") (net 4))
 (segment (start 103.0492 79.740801) (end 102.338 79.740801) (width 0.381) (layer "F.Cu") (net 4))
 (segment (start 94.556 79.558) (end 94.6871 79.558) (width 0.381) (layer "F.Cu") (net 4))
 (segment (start 96.3844 88.9) (end 92.598 88.9) (width 0.381) (layer "F.Cu") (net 4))
 (segment (start 92.456 77.458) (end 94.556 79.558) (width 0.381) (layer "F.Cu") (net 4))
 (segment (start 94.6871 79.558) (end 96.3676 77.8775) (width 0.381) (layer "F.Cu") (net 4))
 (segment (start 103.369199 80.274701) (end 103.5831 80.274701) (width 0.381) (layer "F.Cu") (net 4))
 (segment (start 104.0384 79.819401) (end 103.5831 80.274701) (width 0.381) (layer "F.Cu") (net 4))
 (via (at 97.4852 81.4096) (size 0.8) (drill 0.4) (layers "F.Cu" "B.Cu") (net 4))
 (via (at 99.2124 77.498) (size 0.8) (drill 0.4) (layers "F.Cu" "B.Cu") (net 4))
 (via (at 102.2096 83.2104) (size 0.8) (drill 0.4) (layers "F.Cu" "B.Cu") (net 4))
 (segment (start 95.6336 79.558) (end 94.556 79.558) (width 0.381) (layer "B.Cu") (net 4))
 (segment (start 99.1388 77.5716) (end 96.5424 77.5716) (width 0.381) (layer "B.Cu") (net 4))
 (segment (start 96.5424 77.5716) (end 94.556 79.558) (width 0.381) (layer "B.Cu") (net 4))
 (segment (start 99.2124 77.498) (end 99.1388 77.5716) (width 0.381) (layer "B.Cu") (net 4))
 (segment (start 102.2096 83.2104) (end 100.4088 81.4096) (width 0.381) (layer "B.Cu") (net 4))
 (segment (start 100.4088 81.4096) (end 97.4852 81.4096) (width 0.381) (layer "B.Cu") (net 4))
 (segment (start 97.4852 81.4096) (end 95.6336 79.558) (width 0.381) (layer "B.Cu") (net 4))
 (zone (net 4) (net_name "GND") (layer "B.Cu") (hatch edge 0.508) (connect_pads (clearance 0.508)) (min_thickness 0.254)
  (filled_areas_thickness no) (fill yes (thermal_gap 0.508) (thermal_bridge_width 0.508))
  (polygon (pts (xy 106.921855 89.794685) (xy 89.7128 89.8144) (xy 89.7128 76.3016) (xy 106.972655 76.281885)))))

